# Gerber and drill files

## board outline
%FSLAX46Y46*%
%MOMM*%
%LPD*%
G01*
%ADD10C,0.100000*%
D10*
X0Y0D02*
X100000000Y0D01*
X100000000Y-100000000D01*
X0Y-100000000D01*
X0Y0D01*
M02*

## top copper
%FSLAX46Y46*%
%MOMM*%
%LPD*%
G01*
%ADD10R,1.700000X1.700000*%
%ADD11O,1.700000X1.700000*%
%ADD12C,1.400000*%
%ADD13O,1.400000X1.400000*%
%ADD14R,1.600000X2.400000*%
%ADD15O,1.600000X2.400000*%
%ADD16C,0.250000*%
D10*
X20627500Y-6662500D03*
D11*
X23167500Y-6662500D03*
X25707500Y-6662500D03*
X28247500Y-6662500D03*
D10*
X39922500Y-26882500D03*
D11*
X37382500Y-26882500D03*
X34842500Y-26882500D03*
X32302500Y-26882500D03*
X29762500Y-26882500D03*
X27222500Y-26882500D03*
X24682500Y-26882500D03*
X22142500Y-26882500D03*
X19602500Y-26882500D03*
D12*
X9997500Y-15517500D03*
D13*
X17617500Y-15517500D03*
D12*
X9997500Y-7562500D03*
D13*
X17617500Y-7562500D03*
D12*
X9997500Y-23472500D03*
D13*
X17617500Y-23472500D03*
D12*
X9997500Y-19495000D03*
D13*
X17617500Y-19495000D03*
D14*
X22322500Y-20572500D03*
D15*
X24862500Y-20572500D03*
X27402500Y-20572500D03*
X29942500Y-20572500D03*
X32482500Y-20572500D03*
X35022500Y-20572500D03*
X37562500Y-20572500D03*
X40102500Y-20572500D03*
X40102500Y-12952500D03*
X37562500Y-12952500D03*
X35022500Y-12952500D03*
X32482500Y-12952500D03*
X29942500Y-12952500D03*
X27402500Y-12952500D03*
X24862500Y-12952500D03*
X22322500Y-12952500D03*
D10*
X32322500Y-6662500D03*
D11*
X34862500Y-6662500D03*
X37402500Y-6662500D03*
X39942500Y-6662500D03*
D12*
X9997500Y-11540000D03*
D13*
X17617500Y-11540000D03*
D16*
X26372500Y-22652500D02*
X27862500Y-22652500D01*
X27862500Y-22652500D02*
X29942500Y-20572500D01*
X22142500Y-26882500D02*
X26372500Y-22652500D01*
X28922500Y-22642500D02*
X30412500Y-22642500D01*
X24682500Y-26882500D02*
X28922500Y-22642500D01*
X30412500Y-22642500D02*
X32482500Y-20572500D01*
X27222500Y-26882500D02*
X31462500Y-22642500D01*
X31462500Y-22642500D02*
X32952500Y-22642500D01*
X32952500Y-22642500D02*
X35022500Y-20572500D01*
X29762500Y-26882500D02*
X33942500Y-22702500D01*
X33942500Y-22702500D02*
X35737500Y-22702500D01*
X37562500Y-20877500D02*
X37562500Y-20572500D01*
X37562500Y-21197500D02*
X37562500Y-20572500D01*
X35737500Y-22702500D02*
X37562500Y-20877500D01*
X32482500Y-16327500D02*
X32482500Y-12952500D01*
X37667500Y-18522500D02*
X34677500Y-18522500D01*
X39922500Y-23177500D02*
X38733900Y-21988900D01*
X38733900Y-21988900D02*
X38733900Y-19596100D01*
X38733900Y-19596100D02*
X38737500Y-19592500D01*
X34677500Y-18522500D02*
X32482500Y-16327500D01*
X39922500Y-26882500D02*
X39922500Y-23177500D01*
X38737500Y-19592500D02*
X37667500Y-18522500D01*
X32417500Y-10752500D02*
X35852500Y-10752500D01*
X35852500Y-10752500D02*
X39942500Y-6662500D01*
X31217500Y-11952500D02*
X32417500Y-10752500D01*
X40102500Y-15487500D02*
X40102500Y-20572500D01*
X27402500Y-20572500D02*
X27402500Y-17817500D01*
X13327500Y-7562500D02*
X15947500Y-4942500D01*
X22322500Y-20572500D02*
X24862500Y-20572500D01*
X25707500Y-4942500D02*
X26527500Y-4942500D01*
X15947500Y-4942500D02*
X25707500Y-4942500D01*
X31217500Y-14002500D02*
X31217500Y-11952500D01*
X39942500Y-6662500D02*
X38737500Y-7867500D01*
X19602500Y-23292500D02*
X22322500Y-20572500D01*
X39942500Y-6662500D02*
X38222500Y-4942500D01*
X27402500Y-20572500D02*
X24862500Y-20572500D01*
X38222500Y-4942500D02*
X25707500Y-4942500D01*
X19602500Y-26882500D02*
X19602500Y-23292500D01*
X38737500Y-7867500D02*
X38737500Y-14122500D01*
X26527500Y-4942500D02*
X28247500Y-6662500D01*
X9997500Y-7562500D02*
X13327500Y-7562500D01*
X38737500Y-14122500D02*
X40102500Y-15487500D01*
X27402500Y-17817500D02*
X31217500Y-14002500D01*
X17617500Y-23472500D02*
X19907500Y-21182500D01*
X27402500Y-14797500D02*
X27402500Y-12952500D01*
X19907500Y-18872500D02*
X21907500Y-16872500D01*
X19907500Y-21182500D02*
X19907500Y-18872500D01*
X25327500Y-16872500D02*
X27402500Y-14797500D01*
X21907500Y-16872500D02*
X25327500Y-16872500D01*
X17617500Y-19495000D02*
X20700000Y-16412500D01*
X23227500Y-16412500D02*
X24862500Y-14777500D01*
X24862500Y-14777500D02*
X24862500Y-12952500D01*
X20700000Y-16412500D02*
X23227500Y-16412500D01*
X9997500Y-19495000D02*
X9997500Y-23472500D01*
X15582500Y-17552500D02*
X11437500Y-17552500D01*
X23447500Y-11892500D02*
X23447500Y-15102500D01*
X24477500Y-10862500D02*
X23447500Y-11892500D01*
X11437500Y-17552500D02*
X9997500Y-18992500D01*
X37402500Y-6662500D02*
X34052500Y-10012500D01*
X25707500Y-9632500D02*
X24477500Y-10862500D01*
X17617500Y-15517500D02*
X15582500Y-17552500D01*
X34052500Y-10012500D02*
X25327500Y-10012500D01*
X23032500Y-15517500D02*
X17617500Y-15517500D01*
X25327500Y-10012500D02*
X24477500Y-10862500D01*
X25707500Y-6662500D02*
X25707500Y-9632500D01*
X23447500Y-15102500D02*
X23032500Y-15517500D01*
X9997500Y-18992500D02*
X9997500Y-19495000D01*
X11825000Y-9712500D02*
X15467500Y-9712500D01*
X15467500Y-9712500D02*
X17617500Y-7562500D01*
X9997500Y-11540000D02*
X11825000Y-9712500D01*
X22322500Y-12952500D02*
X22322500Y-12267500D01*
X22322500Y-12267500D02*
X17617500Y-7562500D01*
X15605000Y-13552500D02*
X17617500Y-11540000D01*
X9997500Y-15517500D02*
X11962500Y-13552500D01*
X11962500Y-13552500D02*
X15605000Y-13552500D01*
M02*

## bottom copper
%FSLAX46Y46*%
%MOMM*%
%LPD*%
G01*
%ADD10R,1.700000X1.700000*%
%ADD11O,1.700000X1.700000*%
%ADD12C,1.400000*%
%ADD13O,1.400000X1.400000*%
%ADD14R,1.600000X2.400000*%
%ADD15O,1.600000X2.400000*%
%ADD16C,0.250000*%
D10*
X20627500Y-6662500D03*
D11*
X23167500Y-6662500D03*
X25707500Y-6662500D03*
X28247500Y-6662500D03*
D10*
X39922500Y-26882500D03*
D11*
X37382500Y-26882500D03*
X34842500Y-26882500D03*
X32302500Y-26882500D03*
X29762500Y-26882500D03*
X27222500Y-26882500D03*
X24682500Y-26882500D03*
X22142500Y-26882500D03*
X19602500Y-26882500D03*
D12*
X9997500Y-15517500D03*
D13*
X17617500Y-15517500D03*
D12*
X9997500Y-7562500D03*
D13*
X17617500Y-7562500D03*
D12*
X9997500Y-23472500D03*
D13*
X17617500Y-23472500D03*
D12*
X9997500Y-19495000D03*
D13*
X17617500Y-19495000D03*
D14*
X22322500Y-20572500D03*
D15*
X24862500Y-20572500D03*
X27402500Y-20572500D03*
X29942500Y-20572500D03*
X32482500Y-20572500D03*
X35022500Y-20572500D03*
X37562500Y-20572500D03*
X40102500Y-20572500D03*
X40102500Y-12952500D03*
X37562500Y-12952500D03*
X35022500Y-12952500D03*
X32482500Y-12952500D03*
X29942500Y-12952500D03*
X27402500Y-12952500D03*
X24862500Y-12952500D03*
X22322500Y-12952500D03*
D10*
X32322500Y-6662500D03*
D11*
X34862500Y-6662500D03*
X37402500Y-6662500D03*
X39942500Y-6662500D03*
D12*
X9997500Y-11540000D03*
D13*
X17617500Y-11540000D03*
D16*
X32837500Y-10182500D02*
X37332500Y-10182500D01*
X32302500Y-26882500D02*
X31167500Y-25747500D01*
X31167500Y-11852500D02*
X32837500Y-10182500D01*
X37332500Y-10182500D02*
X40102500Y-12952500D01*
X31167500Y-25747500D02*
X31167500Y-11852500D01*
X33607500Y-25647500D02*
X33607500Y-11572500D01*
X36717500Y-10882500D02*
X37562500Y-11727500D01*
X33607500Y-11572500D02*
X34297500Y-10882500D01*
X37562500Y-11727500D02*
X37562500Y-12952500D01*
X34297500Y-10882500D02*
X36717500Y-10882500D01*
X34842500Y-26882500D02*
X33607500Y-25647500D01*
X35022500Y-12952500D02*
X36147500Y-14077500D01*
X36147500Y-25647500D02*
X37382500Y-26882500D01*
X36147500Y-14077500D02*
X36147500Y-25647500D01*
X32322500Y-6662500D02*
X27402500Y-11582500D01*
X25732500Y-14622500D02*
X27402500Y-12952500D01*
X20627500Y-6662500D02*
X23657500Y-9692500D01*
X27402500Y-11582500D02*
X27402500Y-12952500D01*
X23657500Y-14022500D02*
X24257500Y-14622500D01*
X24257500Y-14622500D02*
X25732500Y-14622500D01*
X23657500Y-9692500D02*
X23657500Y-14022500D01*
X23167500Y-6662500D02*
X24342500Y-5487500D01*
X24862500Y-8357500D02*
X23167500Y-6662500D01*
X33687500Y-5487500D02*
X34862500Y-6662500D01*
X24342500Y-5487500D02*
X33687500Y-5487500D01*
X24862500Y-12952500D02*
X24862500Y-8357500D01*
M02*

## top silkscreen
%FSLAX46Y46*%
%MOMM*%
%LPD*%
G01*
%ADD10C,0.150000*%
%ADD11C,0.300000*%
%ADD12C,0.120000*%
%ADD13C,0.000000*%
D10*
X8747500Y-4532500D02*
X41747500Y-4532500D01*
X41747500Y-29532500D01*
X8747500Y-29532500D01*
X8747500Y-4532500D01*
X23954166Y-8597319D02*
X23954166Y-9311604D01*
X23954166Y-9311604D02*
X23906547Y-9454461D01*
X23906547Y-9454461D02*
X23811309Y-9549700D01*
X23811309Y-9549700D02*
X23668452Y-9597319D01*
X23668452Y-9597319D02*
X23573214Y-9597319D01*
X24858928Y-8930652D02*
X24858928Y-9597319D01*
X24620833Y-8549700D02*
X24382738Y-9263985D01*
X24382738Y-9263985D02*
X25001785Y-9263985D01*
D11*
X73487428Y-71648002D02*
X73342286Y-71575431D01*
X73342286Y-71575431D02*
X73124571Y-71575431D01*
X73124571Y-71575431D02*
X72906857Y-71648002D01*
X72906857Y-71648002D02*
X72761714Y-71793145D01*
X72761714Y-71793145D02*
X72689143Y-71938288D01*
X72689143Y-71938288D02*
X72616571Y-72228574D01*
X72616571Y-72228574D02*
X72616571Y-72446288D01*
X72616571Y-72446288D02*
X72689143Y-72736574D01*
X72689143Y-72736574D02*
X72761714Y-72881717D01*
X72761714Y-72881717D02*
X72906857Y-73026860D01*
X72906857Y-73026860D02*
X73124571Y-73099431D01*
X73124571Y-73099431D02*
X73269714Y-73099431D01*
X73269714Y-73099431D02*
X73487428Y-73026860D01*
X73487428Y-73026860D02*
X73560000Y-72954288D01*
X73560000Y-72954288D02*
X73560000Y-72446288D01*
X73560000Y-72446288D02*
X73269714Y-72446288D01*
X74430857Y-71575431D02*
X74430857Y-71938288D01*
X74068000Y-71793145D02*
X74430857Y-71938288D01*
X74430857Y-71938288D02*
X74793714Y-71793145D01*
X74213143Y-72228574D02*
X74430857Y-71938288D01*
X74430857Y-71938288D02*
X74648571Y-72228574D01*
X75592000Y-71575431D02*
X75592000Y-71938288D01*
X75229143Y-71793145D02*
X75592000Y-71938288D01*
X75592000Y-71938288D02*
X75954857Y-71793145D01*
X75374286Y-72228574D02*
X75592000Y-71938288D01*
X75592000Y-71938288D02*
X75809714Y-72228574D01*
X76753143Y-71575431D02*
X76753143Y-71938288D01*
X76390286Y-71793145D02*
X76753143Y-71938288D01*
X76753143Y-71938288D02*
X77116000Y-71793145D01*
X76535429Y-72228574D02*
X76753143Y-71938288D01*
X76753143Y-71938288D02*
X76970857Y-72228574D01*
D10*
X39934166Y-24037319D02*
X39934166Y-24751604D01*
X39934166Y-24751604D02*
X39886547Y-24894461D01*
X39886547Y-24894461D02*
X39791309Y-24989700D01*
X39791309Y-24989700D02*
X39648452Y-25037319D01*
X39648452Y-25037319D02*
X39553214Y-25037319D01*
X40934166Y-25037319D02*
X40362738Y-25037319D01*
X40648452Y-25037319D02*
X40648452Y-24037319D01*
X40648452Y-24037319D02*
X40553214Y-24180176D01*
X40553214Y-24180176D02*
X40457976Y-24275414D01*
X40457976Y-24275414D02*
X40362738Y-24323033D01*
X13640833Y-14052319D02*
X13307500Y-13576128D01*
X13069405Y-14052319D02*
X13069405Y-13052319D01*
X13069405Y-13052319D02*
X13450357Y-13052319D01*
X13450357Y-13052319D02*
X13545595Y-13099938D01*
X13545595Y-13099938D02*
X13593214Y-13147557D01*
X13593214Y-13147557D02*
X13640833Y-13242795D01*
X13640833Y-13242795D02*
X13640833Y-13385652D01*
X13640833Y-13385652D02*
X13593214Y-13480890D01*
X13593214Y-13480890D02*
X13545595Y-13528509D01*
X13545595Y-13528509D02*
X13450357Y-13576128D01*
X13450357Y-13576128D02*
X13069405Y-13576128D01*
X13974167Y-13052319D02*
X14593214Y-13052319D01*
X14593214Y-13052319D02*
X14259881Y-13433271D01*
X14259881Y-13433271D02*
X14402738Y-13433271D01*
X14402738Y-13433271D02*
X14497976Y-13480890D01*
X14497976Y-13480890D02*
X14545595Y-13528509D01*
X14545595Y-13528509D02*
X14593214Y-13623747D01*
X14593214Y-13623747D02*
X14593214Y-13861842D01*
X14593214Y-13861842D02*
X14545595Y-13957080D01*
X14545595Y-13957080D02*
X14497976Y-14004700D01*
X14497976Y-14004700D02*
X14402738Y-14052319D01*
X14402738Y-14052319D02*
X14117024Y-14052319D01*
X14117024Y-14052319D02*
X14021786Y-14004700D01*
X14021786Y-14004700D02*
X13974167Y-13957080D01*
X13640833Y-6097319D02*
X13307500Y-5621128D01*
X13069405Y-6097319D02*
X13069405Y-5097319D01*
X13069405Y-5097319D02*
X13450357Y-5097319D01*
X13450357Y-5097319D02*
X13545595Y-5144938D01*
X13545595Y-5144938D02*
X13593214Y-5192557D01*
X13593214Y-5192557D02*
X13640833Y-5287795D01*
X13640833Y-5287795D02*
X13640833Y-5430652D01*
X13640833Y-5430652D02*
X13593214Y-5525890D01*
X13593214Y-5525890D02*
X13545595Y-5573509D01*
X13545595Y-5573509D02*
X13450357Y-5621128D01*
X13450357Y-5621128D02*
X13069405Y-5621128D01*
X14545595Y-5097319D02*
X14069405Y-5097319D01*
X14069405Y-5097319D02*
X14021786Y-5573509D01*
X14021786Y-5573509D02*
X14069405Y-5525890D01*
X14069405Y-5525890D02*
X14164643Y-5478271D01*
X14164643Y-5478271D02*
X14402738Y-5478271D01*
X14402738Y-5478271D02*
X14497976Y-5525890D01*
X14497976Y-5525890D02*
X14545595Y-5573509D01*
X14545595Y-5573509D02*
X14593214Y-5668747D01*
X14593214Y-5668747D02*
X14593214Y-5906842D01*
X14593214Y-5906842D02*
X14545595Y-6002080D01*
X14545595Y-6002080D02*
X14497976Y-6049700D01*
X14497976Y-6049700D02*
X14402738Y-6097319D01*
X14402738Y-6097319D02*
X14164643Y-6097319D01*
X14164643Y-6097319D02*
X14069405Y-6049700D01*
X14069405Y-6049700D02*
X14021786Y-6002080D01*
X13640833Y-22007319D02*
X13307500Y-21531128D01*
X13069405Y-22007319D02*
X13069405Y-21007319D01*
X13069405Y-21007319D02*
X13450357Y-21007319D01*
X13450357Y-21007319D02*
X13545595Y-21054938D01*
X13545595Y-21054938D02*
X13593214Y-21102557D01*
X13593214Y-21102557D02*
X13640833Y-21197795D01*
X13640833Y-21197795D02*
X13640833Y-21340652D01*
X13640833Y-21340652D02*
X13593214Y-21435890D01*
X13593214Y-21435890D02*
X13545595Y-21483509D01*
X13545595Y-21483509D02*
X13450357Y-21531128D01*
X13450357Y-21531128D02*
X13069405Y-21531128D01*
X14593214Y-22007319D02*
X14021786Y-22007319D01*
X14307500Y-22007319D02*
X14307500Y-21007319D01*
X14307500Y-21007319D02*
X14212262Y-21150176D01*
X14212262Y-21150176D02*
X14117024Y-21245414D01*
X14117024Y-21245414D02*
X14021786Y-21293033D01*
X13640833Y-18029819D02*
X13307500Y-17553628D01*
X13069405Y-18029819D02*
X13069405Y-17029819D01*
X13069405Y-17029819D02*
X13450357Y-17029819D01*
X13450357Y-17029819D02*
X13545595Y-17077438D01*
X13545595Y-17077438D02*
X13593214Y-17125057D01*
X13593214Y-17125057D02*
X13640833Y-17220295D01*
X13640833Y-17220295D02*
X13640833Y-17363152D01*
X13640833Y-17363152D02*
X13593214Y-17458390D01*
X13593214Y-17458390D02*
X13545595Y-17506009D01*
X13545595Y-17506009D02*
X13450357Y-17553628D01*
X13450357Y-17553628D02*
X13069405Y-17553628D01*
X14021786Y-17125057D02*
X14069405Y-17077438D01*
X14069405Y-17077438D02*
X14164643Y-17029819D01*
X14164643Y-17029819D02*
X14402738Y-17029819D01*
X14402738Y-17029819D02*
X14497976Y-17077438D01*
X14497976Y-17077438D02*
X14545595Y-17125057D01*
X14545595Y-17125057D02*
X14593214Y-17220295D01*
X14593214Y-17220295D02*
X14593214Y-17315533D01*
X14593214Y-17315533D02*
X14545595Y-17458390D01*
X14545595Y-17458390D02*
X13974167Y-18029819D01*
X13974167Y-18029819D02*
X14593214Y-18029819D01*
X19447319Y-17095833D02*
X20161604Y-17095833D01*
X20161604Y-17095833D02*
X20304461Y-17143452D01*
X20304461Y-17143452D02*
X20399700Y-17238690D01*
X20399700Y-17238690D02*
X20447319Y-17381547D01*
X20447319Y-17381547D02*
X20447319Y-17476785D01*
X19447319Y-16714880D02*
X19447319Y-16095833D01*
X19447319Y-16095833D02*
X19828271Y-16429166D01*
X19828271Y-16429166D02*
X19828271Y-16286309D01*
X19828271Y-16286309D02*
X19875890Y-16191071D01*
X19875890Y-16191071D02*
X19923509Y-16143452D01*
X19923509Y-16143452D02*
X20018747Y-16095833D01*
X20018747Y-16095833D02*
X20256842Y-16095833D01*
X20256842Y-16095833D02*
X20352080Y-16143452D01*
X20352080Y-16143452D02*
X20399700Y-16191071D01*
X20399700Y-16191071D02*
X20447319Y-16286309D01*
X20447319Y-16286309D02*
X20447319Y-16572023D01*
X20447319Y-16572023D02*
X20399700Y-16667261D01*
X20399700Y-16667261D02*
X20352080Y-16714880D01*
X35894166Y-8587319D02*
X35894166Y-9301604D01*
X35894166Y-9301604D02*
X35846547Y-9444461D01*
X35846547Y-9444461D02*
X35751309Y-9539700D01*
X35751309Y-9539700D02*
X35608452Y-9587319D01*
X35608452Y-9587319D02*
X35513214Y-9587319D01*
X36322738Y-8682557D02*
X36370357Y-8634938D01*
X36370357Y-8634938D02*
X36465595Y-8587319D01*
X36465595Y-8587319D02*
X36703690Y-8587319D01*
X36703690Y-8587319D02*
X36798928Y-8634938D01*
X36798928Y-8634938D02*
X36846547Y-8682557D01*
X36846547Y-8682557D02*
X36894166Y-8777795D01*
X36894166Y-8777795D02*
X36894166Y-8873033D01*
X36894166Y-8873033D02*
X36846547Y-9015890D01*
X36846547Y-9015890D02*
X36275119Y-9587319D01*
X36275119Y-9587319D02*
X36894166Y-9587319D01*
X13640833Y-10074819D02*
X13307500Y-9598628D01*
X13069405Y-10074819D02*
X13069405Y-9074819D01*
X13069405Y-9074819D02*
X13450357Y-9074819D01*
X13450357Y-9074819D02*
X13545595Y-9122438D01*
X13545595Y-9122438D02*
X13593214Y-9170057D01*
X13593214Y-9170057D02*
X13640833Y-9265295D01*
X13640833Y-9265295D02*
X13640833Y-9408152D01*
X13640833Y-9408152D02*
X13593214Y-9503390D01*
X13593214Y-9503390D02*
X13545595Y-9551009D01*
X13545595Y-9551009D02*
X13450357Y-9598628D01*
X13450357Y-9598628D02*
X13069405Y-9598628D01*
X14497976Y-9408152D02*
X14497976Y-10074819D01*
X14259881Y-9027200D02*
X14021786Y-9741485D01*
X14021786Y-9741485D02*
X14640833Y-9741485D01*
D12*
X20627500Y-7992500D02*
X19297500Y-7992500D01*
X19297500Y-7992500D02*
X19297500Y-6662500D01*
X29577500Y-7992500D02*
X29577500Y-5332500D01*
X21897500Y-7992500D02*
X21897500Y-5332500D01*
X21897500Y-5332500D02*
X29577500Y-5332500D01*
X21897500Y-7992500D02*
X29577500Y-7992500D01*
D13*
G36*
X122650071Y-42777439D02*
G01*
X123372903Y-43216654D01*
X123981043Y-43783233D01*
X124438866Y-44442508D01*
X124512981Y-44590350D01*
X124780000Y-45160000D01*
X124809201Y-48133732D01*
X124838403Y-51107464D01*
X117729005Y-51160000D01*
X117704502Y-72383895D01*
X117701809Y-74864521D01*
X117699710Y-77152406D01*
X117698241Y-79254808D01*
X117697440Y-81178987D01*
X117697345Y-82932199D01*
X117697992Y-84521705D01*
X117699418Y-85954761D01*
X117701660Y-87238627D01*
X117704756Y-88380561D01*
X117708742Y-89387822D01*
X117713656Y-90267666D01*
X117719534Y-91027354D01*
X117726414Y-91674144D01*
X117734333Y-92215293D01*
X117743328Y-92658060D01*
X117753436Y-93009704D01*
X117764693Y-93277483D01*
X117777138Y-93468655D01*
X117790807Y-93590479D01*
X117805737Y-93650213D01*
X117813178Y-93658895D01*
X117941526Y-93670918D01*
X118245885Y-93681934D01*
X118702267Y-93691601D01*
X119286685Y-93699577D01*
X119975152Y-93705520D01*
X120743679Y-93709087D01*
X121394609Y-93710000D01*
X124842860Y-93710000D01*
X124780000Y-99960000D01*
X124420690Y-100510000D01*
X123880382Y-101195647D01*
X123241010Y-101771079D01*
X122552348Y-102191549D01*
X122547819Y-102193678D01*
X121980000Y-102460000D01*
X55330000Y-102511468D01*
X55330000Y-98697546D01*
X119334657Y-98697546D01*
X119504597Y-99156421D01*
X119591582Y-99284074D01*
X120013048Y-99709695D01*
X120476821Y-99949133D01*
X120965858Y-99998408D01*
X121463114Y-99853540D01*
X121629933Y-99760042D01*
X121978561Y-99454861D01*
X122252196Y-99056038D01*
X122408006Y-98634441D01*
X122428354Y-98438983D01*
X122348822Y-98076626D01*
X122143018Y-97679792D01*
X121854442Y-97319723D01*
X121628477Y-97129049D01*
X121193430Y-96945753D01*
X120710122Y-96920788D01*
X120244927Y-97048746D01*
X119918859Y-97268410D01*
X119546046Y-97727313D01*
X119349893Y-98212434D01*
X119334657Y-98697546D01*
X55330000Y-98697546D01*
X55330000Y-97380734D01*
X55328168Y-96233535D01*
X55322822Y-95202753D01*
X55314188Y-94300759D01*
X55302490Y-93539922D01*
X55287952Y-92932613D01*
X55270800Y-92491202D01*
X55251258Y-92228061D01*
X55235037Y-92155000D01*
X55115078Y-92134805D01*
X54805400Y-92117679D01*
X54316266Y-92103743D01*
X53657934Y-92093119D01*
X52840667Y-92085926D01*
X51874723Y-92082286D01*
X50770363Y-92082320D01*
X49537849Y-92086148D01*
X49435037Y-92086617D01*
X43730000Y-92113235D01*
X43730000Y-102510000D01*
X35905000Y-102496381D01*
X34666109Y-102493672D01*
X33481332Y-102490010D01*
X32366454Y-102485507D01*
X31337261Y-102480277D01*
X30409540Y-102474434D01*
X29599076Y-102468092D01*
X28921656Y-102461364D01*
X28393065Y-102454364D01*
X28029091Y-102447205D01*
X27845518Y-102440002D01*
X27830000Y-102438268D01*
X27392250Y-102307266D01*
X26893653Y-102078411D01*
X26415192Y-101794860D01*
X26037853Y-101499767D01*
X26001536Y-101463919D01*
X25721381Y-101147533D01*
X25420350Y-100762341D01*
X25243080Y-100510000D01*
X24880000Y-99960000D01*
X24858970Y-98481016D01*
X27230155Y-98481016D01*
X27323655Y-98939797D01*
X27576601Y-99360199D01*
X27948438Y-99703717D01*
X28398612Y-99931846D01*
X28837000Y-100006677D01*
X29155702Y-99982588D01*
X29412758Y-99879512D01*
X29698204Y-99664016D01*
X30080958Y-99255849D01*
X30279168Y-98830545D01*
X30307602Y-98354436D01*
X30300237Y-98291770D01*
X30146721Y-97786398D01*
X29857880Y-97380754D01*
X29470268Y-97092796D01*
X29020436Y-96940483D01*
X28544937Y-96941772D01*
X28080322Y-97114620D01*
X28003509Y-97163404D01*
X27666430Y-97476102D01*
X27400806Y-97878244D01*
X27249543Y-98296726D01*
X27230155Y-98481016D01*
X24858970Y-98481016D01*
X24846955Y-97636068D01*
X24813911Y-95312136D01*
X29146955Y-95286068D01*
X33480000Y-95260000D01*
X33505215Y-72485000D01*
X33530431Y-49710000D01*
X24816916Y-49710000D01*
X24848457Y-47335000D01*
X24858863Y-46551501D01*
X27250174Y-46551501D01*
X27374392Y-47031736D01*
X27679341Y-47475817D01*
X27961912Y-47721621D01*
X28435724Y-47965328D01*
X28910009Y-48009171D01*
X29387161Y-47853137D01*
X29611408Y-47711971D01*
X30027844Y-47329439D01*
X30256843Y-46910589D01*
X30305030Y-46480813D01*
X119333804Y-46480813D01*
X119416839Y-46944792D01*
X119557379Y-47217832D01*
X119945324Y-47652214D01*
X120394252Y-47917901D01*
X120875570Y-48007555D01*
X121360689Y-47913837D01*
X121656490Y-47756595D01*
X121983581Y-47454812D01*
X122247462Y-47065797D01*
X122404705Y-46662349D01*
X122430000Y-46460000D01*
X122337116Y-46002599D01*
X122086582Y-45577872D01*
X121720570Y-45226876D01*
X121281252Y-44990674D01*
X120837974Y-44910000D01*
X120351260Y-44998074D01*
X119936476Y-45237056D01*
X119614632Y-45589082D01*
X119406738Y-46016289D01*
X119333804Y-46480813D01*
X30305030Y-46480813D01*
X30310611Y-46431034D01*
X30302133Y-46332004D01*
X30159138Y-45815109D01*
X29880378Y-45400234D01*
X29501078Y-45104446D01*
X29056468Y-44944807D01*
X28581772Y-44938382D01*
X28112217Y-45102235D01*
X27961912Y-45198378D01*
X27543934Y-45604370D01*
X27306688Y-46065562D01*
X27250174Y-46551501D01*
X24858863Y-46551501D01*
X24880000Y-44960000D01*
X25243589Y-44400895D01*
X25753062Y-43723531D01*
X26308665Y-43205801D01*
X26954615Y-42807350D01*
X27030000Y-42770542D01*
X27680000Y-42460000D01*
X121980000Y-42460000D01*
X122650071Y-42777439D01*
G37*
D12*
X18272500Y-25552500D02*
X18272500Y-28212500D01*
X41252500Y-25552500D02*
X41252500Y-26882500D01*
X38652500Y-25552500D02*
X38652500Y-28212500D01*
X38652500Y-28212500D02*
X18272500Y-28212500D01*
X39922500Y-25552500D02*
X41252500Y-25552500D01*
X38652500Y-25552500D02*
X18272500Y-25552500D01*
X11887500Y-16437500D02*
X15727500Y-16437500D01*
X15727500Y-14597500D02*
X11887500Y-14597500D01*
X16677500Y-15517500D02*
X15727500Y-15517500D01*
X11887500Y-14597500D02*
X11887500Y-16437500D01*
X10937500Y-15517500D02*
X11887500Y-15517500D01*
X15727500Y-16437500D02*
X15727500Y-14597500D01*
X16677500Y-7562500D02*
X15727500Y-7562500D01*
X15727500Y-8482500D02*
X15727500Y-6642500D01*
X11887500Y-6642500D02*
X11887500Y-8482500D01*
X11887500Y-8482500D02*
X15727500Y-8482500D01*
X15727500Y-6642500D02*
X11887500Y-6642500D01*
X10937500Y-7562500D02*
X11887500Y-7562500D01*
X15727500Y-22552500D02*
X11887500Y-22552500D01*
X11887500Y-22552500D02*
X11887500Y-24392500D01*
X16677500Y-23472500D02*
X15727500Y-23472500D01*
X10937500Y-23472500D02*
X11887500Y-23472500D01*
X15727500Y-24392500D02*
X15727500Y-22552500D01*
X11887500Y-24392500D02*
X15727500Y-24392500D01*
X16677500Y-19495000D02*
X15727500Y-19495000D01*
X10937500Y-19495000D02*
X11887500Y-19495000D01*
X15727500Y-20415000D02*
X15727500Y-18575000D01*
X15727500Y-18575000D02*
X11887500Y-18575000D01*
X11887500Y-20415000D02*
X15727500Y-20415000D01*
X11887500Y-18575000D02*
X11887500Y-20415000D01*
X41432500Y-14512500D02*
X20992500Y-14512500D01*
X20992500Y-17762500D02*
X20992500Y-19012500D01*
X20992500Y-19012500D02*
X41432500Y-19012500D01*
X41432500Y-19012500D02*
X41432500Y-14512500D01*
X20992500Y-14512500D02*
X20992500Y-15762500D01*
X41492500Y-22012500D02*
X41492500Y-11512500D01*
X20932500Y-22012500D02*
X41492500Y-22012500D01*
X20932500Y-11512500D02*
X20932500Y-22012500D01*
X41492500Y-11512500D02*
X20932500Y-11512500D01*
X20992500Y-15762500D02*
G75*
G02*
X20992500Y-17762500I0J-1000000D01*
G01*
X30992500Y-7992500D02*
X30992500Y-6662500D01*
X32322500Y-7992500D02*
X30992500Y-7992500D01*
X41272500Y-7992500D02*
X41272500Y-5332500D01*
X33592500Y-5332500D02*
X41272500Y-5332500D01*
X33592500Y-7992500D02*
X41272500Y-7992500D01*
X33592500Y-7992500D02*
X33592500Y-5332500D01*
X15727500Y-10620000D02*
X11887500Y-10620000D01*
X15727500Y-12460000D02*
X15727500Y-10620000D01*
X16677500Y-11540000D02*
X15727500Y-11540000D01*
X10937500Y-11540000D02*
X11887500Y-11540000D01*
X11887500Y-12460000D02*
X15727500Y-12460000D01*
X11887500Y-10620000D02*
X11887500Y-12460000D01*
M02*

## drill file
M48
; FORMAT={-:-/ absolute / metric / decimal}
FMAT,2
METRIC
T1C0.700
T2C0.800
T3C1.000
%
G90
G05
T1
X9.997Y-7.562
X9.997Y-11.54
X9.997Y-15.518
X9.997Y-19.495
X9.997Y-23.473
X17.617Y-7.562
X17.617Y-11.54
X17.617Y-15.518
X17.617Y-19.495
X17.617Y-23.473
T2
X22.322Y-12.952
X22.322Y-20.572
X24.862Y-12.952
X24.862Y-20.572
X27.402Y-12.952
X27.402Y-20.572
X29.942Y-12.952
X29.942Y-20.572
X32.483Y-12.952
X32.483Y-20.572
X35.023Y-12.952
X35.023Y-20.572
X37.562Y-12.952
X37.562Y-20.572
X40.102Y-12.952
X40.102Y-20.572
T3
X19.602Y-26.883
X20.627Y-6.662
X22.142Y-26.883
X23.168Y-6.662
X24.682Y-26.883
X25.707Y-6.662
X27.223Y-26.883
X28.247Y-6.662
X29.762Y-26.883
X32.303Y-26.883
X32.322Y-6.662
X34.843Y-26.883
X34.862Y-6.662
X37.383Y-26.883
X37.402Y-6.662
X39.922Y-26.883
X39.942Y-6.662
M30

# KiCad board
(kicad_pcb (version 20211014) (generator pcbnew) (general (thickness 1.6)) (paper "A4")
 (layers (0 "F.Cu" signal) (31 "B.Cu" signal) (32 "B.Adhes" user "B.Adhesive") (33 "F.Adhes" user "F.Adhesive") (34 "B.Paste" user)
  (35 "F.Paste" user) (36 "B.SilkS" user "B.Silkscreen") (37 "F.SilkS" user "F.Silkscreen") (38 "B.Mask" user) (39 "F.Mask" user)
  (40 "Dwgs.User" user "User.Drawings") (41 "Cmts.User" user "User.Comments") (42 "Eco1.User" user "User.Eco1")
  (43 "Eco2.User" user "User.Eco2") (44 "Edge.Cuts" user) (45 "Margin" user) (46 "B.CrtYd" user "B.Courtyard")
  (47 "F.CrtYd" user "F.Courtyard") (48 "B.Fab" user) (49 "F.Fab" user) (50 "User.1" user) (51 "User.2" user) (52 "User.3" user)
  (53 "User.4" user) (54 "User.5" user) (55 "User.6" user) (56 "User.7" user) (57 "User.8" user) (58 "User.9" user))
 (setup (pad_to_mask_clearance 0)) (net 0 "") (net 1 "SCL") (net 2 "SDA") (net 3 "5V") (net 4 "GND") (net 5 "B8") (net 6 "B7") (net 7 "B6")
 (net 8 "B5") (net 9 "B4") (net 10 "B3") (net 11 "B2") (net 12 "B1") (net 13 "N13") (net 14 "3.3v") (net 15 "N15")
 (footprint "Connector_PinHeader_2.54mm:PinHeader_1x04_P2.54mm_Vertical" (layer "F.Cu") (at 20.6275 6.6625 90)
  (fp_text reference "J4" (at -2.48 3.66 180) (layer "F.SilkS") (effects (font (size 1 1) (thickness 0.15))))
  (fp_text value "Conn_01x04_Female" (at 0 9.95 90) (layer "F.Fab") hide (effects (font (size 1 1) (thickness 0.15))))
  (fp_line (start -1.33 0) (end -1.33 -1.33) (layer "F.SilkS") (width 0.12))
  (fp_line (start -1.33 -1.33) (end 0 -1.33) (layer "F.SilkS") (width 0.12))
  (fp_line (start -1.33 8.95) (end 1.33 8.95) (layer "F.SilkS") (width 0.12))
  (fp_line (start -1.33 1.27) (end 1.33 1.27) (layer "F.SilkS") (width 0.12))
  (fp_line (start 1.33 1.27) (end 1.33 8.95) (layer "F.SilkS") (width 0.12))
  (fp_line (start -1.33 1.27) (end -1.33 8.95) (layer "F.SilkS") (width 0.12))
  (pad "1" thru_hole rect (at 0 0 90) (size 1.7 1.7) (drill 1) (layers *.Cu *.Mask) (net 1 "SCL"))
  (pad "2" thru_hole oval (at 0 2.54 90) (size 1.7 1.7) (drill 1) (layers *.Cu *.Mask) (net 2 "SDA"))
  (pad "3" thru_hole oval (at 0 5.08 90) (size 1.7 1.7) (drill 1) (layers *.Cu *.Mask) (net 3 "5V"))
  (pad "4" thru_hole oval (at 0 7.62 90) (size 1.7 1.7) (drill 1) (layers *.Cu *.Mask) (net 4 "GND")))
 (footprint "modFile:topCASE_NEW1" (layer "F.Cu") (at 74.83 72.41)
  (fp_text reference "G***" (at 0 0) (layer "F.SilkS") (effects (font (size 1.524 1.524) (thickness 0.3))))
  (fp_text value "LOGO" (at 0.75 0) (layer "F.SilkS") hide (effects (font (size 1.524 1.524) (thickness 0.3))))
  (fp_poly
   (pts (xy 47.820071 -29.632561) (xy 48.542903 -29.193346) (xy 49.151043 -28.626767) (xy 49.608866 -27.967492) (xy 49.682981 -27.81965)
    (xy 49.95 -27.25) (xy 49.979201 -24.276268) (xy 50.008403 -21.302536) (xy 42.899005 -21.25) (xy 42.874502 -0.026105)
    (xy 42.871809 2.454521) (xy 42.86971 4.742406) (xy 42.868241 6.844808) (xy 42.86744 8.768987) (xy 42.867345 10.522199)
    (xy 42.867992 12.111705) (xy 42.869418 13.544761) (xy 42.87166 14.828627) (xy 42.874756 15.970561) (xy 42.878742 16.977822)
    (xy 42.883656 17.857666) (xy 42.889534 18.617354) (xy 42.896414 19.264144) (xy 42.904333 19.805293) (xy 42.913328 20.24806)
    (xy 42.923436 20.599704) (xy 42.934693 20.867483) (xy 42.947138 21.058655) (xy 42.960807 21.180479) (xy 42.975737 21.240213)
    (xy 42.983178 21.248895) (xy 43.111526 21.260918) (xy 43.415885 21.271934) (xy 43.872267 21.281601) (xy 44.456685 21.289577)
    (xy 45.145152 21.29552) (xy 45.913679 21.299087) (xy 46.564609 21.3) (xy 50.01286 21.3) (xy 49.95 27.55) (xy 49.59069 28.1)
    (xy 49.050382 28.785647) (xy 48.41101 29.361079) (xy 47.722348 29.781549) (xy 47.717819 29.783678) (xy 47.15 30.05) (xy -19.5 30.101468)
    (xy -19.5 26.287546) (xy 44.504657 26.287546) (xy 44.674597 26.746421) (xy 44.761582 26.874074) (xy 45.183048 27.299695)
    (xy 45.646821 27.539133) (xy 46.135858 27.588408) (xy 46.633114 27.44354) (xy 46.799933 27.350042) (xy 47.148561 27.044861)
    (xy 47.422196 26.646038) (xy 47.578006 26.224441) (xy 47.598354 26.028983) (xy 47.518822 25.666626) (xy 47.313018 25.269792)
    (xy 47.024442 24.909723) (xy 46.798477 24.719049) (xy 46.36343 24.535753) (xy 45.880122 24.510788) (xy 45.414927 24.638746)
    (xy 45.088859 24.85841) (xy 44.716046 25.317313) (xy 44.519893 25.802434) (xy 44.504657 26.287546) (xy -19.5 26.287546)
    (xy -19.5 24.970734) (xy -19.501832 23.823535) (xy -19.507178 22.792753) (xy -19.515812 21.890759) (xy -19.52751 21.129922)
    (xy -19.542048 20.522613) (xy -19.5592 20.081202) (xy -19.578742 19.818061) (xy -19.594963 19.745) (xy -19.714922 19.724805)
    (xy -20.0246 19.707679) (xy -20.513734 19.693743) (xy -21.172066 19.683119) (xy -21.989333 19.675926) (xy -22.955277 19.672286)
    (xy -24.059637 19.67232) (xy -25.292151 19.676148) (xy -25.394963 19.676617) (xy -31.1 19.703235) (xy -31.1 30.1) (xy -38.925 30.086381)
    (xy -40.163891 30.083672) (xy -41.348668 30.08001) (xy -42.463546 30.075507) (xy -43.492739 30.070277) (xy -44.42046 30.064434)
    (xy -45.230924 30.058092) (xy -45.908344 30.051364) (xy -46.436935 30.044364) (xy -46.800909 30.037205) (xy -46.984482 30.030002)
    (xy -47 30.028268) (xy -47.43775 29.897266) (xy -47.936347 29.668411) (xy -48.414808 29.38486) (xy -48.792147 29.089767)
    (xy -48.828464 29.053919) (xy -49.108619 28.737533) (xy -49.40965 28.352341) (xy -49.58692 28.1) (xy -49.95 27.55)
    (xy -49.97103 26.071016) (xy -47.599845 26.071016) (xy -47.506345 26.529797) (xy -47.253399 26.950199) (xy -46.881562 27.293717)
    (xy -46.431388 27.521846) (xy -45.993 27.596677) (xy -45.674298 27.572588) (xy -45.417242 27.469512) (xy -45.131796 27.254016)
    (xy -44.749042 26.845849) (xy -44.550832 26.420545) (xy -44.522398 25.944436) (xy -44.529763 25.88177) (xy -44.683279 25.376398)
    (xy -44.97212 24.970754) (xy -45.359732 24.682796) (xy -45.809564 24.530483) (xy -46.285063 24.531772) (xy -46.749678 24.70462)
    (xy -46.826491 24.753404) (xy -47.16357 25.066102) (xy -47.429194 25.468244) (xy -47.580457 25.886726) (xy -47.599845 26.071016)
    (xy -49.97103 26.071016) (xy -49.983045 25.226068) (xy -50.016089 22.902136) (xy -45.683045 22.876068) (xy -41.35 22.85)
    (xy -41.324785 0.075) (xy -41.299569 -22.7) (xy -50.013084 -22.7) (xy -49.981543 -25.075) (xy -49.971137 -25.858499)
    (xy -47.579826 -25.858499) (xy -47.455608 -25.378264) (xy -47.150659 -24.934183) (xy -46.868088 -24.688379) (xy -46.394276 -24.444672)
    (xy -45.919991 -24.400829) (xy -45.442839 -24.556863) (xy -45.218592 -24.698029) (xy -44.802156 -25.080561) (xy -44.573157 -25.499411)
    (xy -44.52497 -25.929187) (xy 44.503804 -25.929187) (xy 44.586839 -25.465208) (xy 44.727379 -25.192168) (xy 45.115324 -24.757786)
    (xy 45.564252 -24.492099) (xy 46.04557 -24.402445) (xy 46.530689 -24.496163) (xy 46.82649 -24.653405) (xy 47.153581 -24.955188)
    (xy 47.417462 -25.344203) (xy 47.574705 -25.747651) (xy 47.6 -25.95) (xy 47.507116 -26.407401) (xy 47.256582 -26.832128)
    (xy 46.89057 -27.183124) (xy 46.451252 -27.419326) (xy 46.007974 -27.5) (xy 45.52126 -27.411926) (xy 45.106476 -27.172944)
    (xy 44.784632 -26.820918) (xy 44.576738 -26.393711) (xy 44.503804 -25.929187) (xy -44.52497 -25.929187) (xy -44.519389 -25.978966)
    (xy -44.527867 -26.077996) (xy -44.670862 -26.594891) (xy -44.949622 -27.009766) (xy -45.328922 -27.305554) (xy -45.773532 -27.465193)
    (xy -46.248228 -27.471618) (xy -46.717783 -27.307765) (xy -46.868088 -27.211622) (xy -47.286066 -26.80563) (xy -47.523312 -26.344438)
    (xy -47.579826 -25.858499) (xy -49.971137 -25.858499) (xy -49.95 -27.45) (xy -49.586411 -28.009105) (xy -49.076938 -28.686469)
    (xy -48.521335 -29.204199) (xy -47.875385 -29.60265) (xy -47.8 -29.639458) (xy -47.15 -29.95) (xy 47.15 -29.95))
   (layer "F.SilkS") (width 0) (fill solid)))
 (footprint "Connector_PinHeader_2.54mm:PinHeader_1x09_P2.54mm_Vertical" (layer "F.Cu") (at 39.9225 26.8825 -90)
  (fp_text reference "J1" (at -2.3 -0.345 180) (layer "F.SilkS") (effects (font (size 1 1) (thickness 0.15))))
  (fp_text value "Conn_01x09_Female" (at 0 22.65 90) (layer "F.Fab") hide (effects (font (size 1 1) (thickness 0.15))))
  (fp_line (start -1.33 21.65) (end 1.33 21.65) (layer "F.SilkS") (width 0.12))
  (fp_line (start -1.33 -1.33) (end 0 -1.33) (layer "F.SilkS") (width 0.12))
  (fp_line (start -1.33 1.27) (end 1.33 1.27) (layer "F.SilkS") (width 0.12))
  (fp_line (start 1.33 1.27) (end 1.33 21.65) (layer "F.SilkS") (width 0.12))
  (fp_line (start -1.33 0) (end -1.33 -1.33) (layer "F.SilkS") (width 0.12))
  (fp_line (start -1.33 1.27) (end -1.33 21.65) (layer "F.SilkS") (width 0.12))
  (pad "1" thru_hole rect (at 0 0 270) (size 1.7 1.7) (drill 1) (layers *.Cu *.Mask) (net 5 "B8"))
  (pad "2" thru_hole oval (at 0 2.54 270) (size 1.7 1.7) (drill 1) (layers *.Cu *.Mask) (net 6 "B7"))
  (pad "3" thru_hole oval (at 0 5.08 270) (size 1.7 1.7) (drill 1) (layers *.Cu *.Mask) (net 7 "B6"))
  (pad "4" thru_hole oval (at 0 7.62 270) (size 1.7 1.7) (drill 1) (layers *.Cu *.Mask) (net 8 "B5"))
  (pad "5" thru_hole oval (at 0 10.16 270) (size 1.7 1.7) (drill 1) (layers *.Cu *.Mask) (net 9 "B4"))
  (pad "6" thru_hole oval (at 0 12.7 270) (size 1.7 1.7) (drill 1) (layers *.Cu *.Mask) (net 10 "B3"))
  (pad "7" thru_hole oval (at 0 15.24 270) (size 1.7 1.7) (drill 1) (layers *.Cu *.Mask) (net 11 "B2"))
  (pad "8" thru_hole oval (at 0 17.78 270) (size 1.7 1.7) (drill 1) (layers *.Cu *.Mask) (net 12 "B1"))
  (pad "9" thru_hole oval (at 0 20.32 270) (size 1.7 1.7) (drill 1) (layers *.Cu *.Mask) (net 4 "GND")))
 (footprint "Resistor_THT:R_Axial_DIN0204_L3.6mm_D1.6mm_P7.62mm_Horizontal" (layer "F.Cu") (at 9.9975 15.5175)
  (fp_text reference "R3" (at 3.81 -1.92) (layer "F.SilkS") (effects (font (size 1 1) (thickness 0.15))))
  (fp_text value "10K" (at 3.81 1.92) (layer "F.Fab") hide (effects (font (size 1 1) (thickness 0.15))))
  (fp_line (start 1.89 0.92) (end 5.73 0.92) (layer "F.SilkS") (width 0.12))
  (fp_line (start 5.73 -0.92) (end 1.89 -0.92) (layer "F.SilkS") (width 0.12))
  (fp_line (start 6.68 0) (end 5.73 0) (layer "F.SilkS") (width 0.12))
  (fp_line (start 1.89 -0.92) (end 1.89 0.92) (layer "F.SilkS") (width 0.12))
  (fp_line (start 0.94 0) (end 1.89 0) (layer "F.SilkS") (width 0.12))
  (fp_line (start 5.73 0.92) (end 5.73 -0.92) (layer "F.SilkS") (width 0.12))
  (pad "1" thru_hole circle (at 0 0) (size 1.4 1.4) (drill 0.7) (layers *.Cu *.Mask) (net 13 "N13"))
  (pad "2" thru_hole oval (at 7.62 0) (size 1.4 1.4) (drill 0.7) (layers *.Cu *.Mask) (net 3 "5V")))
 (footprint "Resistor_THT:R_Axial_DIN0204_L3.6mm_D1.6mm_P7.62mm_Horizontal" (layer "F.Cu") (at 9.9975 7.5625)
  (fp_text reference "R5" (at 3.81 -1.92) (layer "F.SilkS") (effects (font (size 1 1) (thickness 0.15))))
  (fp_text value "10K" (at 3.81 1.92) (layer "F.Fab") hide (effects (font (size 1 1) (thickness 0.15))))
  (fp_line (start 6.68 0) (end 5.73 0) (layer "F.SilkS") (width 0.12))
  (fp_line (start 5.73 0.92) (end 5.73 -0.92) (layer "F.SilkS") (width 0.12))
  (fp_line (start 1.89 -0.92) (end 1.89 0.92) (layer "F.SilkS") (width 0.12))
  (fp_line (start 1.89 0.92) (end 5.73 0.92) (layer "F.SilkS") (width 0.12))
  (fp_line (start 5.73 -0.92) (end 1.89 -0.92) (layer "F.SilkS") (width 0.12))
  (fp_line (start 0.94 0) (end 1.89 0) (layer "F.SilkS") (width 0.12))
  (pad "1" thru_hole circle (at 0 0) (size 1.4 1.4) (drill 0.7) (layers *.Cu *.Mask) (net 4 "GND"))
  (pad "2" thru_hole oval (at 7.62 0) (size 1.4 1.4) (drill 0.7) (layers *.Cu *.Mask) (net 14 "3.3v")))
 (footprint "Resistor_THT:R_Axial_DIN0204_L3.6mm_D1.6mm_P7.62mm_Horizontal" (layer "F.Cu") (at 9.9975 23.4725)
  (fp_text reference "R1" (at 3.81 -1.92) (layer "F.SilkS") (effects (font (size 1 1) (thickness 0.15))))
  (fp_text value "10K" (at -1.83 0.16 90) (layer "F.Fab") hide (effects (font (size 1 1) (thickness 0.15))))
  (fp_line (start 5.73 -0.92) (end 1.89 -0.92) (layer "F.SilkS") (width 0.12))
  (fp_line (start 1.89 -0.92) (end 1.89 0.92) (layer "F.SilkS") (width 0.12))
  (fp_line (start 6.68 0) (end 5.73 0) (layer "F.SilkS") (width 0.12))
  (fp_line (start 0.94 0) (end 1.89 0) (layer "F.SilkS") (width 0.12))
  (fp_line (start 5.73 0.92) (end 5.73 -0.92) (layer "F.SilkS") (width 0.12))
  (fp_line (start 1.89 0.92) (end 5.73 0.92) (layer "F.SilkS") (width 0.12))
  (pad "1" thru_hole circle (at 0 0) (size 1.4 1.4) (drill 0.7) (layers *.Cu *.Mask) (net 3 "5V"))
  (pad "2" thru_hole oval (at 7.62 0) (size 1.4 1.4) (drill 0.7) (layers *.Cu *.Mask) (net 1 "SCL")))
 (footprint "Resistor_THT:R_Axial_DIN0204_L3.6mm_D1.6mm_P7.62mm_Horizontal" (layer "F.Cu") (at 9.9975 19.495)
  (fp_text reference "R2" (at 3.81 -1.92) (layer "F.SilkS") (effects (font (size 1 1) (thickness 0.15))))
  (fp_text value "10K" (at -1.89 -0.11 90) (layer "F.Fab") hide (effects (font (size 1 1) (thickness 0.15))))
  (fp_line (start 6.68 0) (end 5.73 0) (layer "F.SilkS") (width 0.12))
  (fp_line (start 0.94 0) (end 1.89 0) (layer "F.SilkS") (width 0.12))
  (fp_line (start 5.73 0.92) (end 5.73 -0.92) (layer "F.SilkS") (width 0.12))
  (fp_line (start 5.73 -0.92) (end 1.89 -0.92) (layer "F.SilkS") (width 0.12))
  (fp_line (start 1.89 0.92) (end 5.73 0.92) (layer "F.SilkS") (width 0.12))
  (fp_line (start 1.89 -0.92) (end 1.89 0.92) (layer "F.SilkS") (width 0.12))
  (pad "1" thru_hole circle (at 0 0) (size 1.4 1.4) (drill 0.7) (layers *.Cu *.Mask) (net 3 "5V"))
  (pad "2" thru_hole oval (at 7.62 0) (size 1.4 1.4) (drill 0.7) (layers *.Cu *.Mask) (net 2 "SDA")))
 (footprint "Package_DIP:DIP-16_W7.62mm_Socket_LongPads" (layer "F.Cu") (at 22.3225 20.5725 90)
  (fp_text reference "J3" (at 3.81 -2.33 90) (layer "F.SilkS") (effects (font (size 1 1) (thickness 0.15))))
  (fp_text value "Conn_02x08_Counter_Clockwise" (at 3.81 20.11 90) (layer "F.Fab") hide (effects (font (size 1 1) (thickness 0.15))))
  (fp_line (start 6.06 19.11) (end 6.06 -1.33) (layer "F.SilkS") (width 0.12))
  (fp_line (start 2.81 -1.33) (end 1.56 -1.33) (layer "F.SilkS") (width 0.12))
  (fp_line (start 1.56 -1.33) (end 1.56 19.11) (layer "F.SilkS") (width 0.12))
  (fp_line (start 1.56 19.11) (end 6.06 19.11) (layer "F.SilkS") (width 0.12))
  (fp_line (start 6.06 -1.33) (end 4.81 -1.33) (layer "F.SilkS") (width 0.12))
  (fp_line (start -1.44 19.17) (end 9.06 19.17) (layer "F.SilkS") (width 0.12))
  (fp_line (start -1.44 -1.39) (end -1.44 19.17) (layer "F.SilkS") (width 0.12))
  (fp_line (start 9.06 -1.39) (end -1.44 -1.39) (layer "F.SilkS") (width 0.12))
  (fp_line (start 9.06 19.17) (end 9.06 -1.39) (layer "F.SilkS") (width 0.12))
  (fp_arc (start 4.81 -1.33) (mid 3.81 -0.33) (end 2.81 -1.33) (layer "F.SilkS") (width 0.12))
  (pad "1" thru_hole rect (at 0 0 90) (size 2.4 1.6) (drill 0.8) (layers *.Cu *.Mask) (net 4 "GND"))
  (pad "2" thru_hole oval (at 0 2.54 90) (size 2.4 1.6) (drill 0.8) (layers *.Cu *.Mask) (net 4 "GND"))
  (pad "3" thru_hole oval (at 0 5.08 90) (size 2.4 1.6) (drill 0.8) (layers *.Cu *.Mask) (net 4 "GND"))
  (pad "4" thru_hole oval (at 0 7.62 90) (size 2.4 1.6) (drill 0.8) (layers *.Cu *.Mask) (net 12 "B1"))
  (pad "5" thru_hole oval (at 0 10.16 90) (size 2.4 1.6) (drill 0.8) (layers *.Cu *.Mask) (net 11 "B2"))
  (pad "6" thru_hole oval (at 0 12.7 90) (size 2.4 1.6) (drill 0.8) (layers *.Cu *.Mask) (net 10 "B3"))
  (pad "7" thru_hole oval (at 0 15.24 90) (size 2.4 1.6) (drill 0.8) (layers *.Cu *.Mask) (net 9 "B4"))
  (pad "8" thru_hole oval (at 0 17.78 90) (size 2.4 1.6) (drill 0.8) (layers *.Cu *.Mask) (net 4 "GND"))
  (pad "9" thru_hole oval (at 7.62 17.78 90) (size 2.4 1.6) (drill 0.8) (layers *.Cu *.Mask) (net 8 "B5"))
  (pad "10" thru_hole oval (at 7.62 15.24 90) (size 2.4 1.6) (drill 0.8) (layers *.Cu *.Mask) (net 7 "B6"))
  (pad "11" thru_hole oval (at 7.62 12.7 90) (size 2.4 1.6) (drill 0.8) (layers *.Cu *.Mask) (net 6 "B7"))
  (pad "12" thru_hole oval (at 7.62 10.16 90) (size 2.4 1.6) (drill 0.8) (layers *.Cu *.Mask) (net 5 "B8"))
  (pad "13" thru_hole oval (at 7.62 7.62 90) (size 2.4 1.6) (drill 0.8) (layers *.Cu *.Mask) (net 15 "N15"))
  (pad "14" thru_hole oval (at 7.62 5.08 90) (size 2.4 1.6) (drill 0.8) (layers *.Cu *.Mask) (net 1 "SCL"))
  (pad "15" thru_hole oval (at 7.62 2.54 90) (size 2.4 1.6) (drill 0.8) (layers *.Cu *.Mask) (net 2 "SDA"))
  (pad "16" thru_hole oval (at 7.62 0 90) (size 2.4 1.6) (drill 0.8) (layers *.Cu *.Mask) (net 14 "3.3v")))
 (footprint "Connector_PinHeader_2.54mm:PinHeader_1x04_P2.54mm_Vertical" (layer "F.Cu") (at 32.3225 6.6625 90)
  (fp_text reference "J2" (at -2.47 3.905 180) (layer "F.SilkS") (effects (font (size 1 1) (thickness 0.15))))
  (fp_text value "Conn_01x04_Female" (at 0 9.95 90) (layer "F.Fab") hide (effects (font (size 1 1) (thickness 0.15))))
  (fp_line (start -1.33 -1.33) (end 0 -1.33) (layer "F.SilkS") (width 0.12))
  (fp_line (start -1.33 0) (end -1.33 -1.33) (layer "F.SilkS") (width 0.12))
  (fp_line (start -1.33 8.95) (end 1.33 8.95) (layer "F.SilkS") (width 0.12))
  (fp_line (start 1.33 1.27) (end 1.33 8.95) (layer "F.SilkS") (width 0.12))
  (fp_line (start -1.33 1.27) (end -1.33 8.95) (layer "F.SilkS") (width 0.12))
  (fp_line (start -1.33 1.27) (end 1.33 1.27) (layer "F.SilkS") (width 0.12))
  (pad "1" thru_hole rect (at 0 0 90) (size 1.7 1.7) (drill 1) (layers *.Cu *.Mask) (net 1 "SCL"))
  (pad "2" thru_hole oval (at 0 2.54 90) (size 1.7 1.7) (drill 1) (layers *.Cu *.Mask) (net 2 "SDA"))
  (pad "3" thru_hole oval (at 0 5.08 90) (size 1.7 1.7) (drill 1) (layers *.Cu *.Mask) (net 3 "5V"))
  (pad "4" thru_hole oval (at 0 7.62 90) (size 1.7 1.7) (drill 1) (layers *.Cu *.Mask) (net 4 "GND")))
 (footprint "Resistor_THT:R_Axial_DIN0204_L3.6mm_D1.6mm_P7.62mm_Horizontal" (layer "F.Cu") (at 9.9975 11.54)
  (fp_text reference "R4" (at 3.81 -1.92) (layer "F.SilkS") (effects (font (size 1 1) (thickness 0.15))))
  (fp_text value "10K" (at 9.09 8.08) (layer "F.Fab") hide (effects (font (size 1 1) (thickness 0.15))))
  (fp_line (start 5.73 -0.92) (end 1.89 -0.92) (layer "F.SilkS") (width 0.12))
  (fp_line (start 5.73 0.92) (end 5.73 -0.92) (layer "F.SilkS") (width 0.12))
  (fp_line (start 6.68 0) (end 5.73 0) (layer "F.SilkS") (width 0.12))
  (fp_line (start 0.94 0) (end 1.89 0) (layer "F.SilkS") (width 0.12))
  (fp_line (start 1.89 0.92) (end 5.73 0.92) (layer "F.SilkS") (width 0.12))
  (fp_line (start 1.89 -0.92) (end 1.89 0.92) (layer "F.SilkS") (width 0.12))
  (pad "1" thru_hole circle (at 0 0) (size 1.4 1.4) (drill 0.7) (layers *.Cu *.Mask) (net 14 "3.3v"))
  (pad "2" thru_hole oval (at 7.62 0) (size 1.4 1.4) (drill 0.7) (layers *.Cu *.Mask) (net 13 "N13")))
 (gr_rect (start 41.7475 29.5325) (end 8.7475 4.5325) (layer "F.SilkS") (width 0.15) (fill none))
 (gr_rect (start 0 0) (end 100 100) (layer "Edge.Cuts") (width 0.1) (fill none))
 (segment (start 26.3725 22.6525) (end 27.8625 22.6525) (width 0.25) (layer "F.Cu") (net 12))
 (segment (start 27.8625 22.6525) (end 29.9425 20.5725) (width 0.25) (layer "F.Cu") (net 12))
 (segment (start 22.1425 26.8825) (end 26.3725 22.6525) (width 0.25) (layer "F.Cu") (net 12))
 (segment (start 28.9225 22.6425) (end 30.4125 22.6425) (width 0.25) (layer "F.Cu") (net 11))
 (segment (start 24.6825 26.8825) (end 28.9225 22.6425) (width 0.25) (layer "F.Cu") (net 11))
 (segment (start 30.4125 22.6425) (end 32.4825 20.5725) (width 0.25) (layer "F.Cu") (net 11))
 (segment (start 27.2225 26.8825) (end 31.4625 22.6425) (width 0.25) (layer "F.Cu") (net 10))
 (segment (start 31.4625 22.6425) (end 32.9525 22.6425) (width 0.25) (layer "F.Cu") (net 10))
 (segment (start 32.9525 22.6425) (end 35.0225 20.5725) (width 0.25) (layer "F.Cu") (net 10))
 (segment (start 29.7625 26.8825) (end 33.9425 22.7025) (width 0.25) (layer "F.Cu") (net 9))
 (segment (start 33.9425 22.7025) (end 35.7375 22.7025) (width 0.25) (layer "F.Cu") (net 9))
 (segment (start 37.5625 20.8775) (end 37.5625 20.5725) (width 0.25) (layer "F.Cu") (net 9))
 (segment (start 37.5625 21.1975) (end 37.5625 20.5725) (width 0.25) (layer "F.Cu") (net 9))
 (segment (start 35.7375 22.7025) (end 37.5625 20.8775) (width 0.25) (layer "F.Cu") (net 9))
 (segment (start 32.8375 10.1825) (end 37.3325 10.1825) (width 0.25) (layer "B.Cu") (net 8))
 (segment (start 32.3025 26.8825) (end 31.1675 25.7475) (width 0.25) (layer "B.Cu") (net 8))
 (segment (start 31.1675 11.8525) (end 32.8375 10.1825) (width 0.25) (layer "B.Cu") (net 8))
 (segment (start 37.3325 10.1825) (end 40.1025 12.9525) (width 0.25) (layer "B.Cu") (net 8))
 (segment (start 31.1675 25.7475) (end 31.1675 11.8525) (width 0.25) (layer "B.Cu") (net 8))
 (segment (start 33.6075 25.6475) (end 33.6075 11.5725) (width 0.25) (layer "B.Cu") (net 7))
 (segment (start 36.7175 10.8825) (end 37.5625 11.7275) (width 0.25) (layer "B.Cu") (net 7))
 (segment (start 33.6075 11.5725) (end 34.2975 10.8825) (width 0.25) (layer "B.Cu") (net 7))
 (segment (start 37.5625 11.7275) (end 37.5625 12.9525) (width 0.25) (layer "B.Cu") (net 7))
 (segment (start 34.2975 10.8825) (end 36.7175 10.8825) (width 0.25) (layer "B.Cu") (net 7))
 (segment (start 34.8425 26.8825) (end 33.6075 25.6475) (width 0.25) (layer "B.Cu") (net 7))
 (segment (start 35.0225 12.9525) (end 36.1475 14.0775) (width 0.25) (layer "B.Cu") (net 6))
 (segment (start 36.1475 25.6475) (end 37.3825 26.8825) (width 0.25) (layer "B.Cu") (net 6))
 (segment (start 36.1475 14.0775) (end 36.1475 25.6475) (width 0.25) (layer "B.Cu") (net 6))
 (segment (start 32.4825 16.3275) (end 32.4825 12.9525) (width 0.25) (layer "F.Cu") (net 5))
 (segment (start 37.6675 18.5225) (end 34.6775 18.5225) (width 0.25) (layer "F.Cu") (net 5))
 (segment (start 39.9225 23.1775) (end 38.7339 21.9889) (width 0.25) (layer "F.Cu") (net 5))
 (segment (start 38.7339 21.9889) (end 38.7339 19.5961) (width 0.25) (layer "F.Cu") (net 5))
 (segment (start 38.7339 19.5961) (end 38.7375 19.5925) (width 0.25) (layer "F.Cu") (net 5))
 (segment (start 34.6775 18.5225) (end 32.4825 16.3275) (width 0.25) (layer "F.Cu") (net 5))
 (segment (start 39.9225 26.8825) (end 39.9225 23.1775) (width 0.25) (layer "F.Cu") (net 5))
 (segment (start 38.7375 19.5925) (end 37.6675 18.5225) (width 0.25) (layer "F.Cu") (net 5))
 (segment (start 32.4175 10.7525) (end 35.8525 10.7525) (width 0.25) (layer "F.Cu") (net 4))
 (segment (start 35.8525 10.7525) (end 39.9425 6.6625) (width 0.25) (layer "F.Cu") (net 4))
 (segment (start 31.2175 11.9525) (end 32.4175 10.7525) (width 0.25) (layer "F.Cu") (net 4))
 (segment (start 40.1025 15.4875) (end 40.1025 20.5725) (width 0.25) (layer "F.Cu") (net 4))
 (segment (start 27.4025 20.5725) (end 27.4025 17.8175) (width 0.25) (layer "F.Cu") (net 4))
 (segment (start 13.3275 7.5625) (end 15.9475 4.9425) (width 0.25) (layer "F.Cu") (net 4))
 (segment (start 22.3225 20.5725) (end 24.8625 20.5725) (width 0.25) (layer "F.Cu") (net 4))
 (segment (start 25.7075 4.9425) (end 26.5275 4.9425) (width 0.25) (layer "F.Cu") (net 4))
 (segment (start 15.9475 4.9425) (end 25.7075 4.9425) (width 0.25) (layer "F.Cu") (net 4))
 (segment (start 31.2175 14.0025) (end 31.2175 11.9525) (width 0.25) (layer "F.Cu") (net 4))
 (segment (start 39.9425 6.6625) (end 38.7375 7.8675) (width 0.25) (layer "F.Cu") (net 4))
 (segment (start 19.6025 23.2925) (end 22.3225 20.5725) (width 0.25) (layer "F.Cu") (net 4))
 (segment (start 39.9425 6.6625) (end 38.2225 4.9425) (width 0.25) (layer "F.Cu") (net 4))
 (segment (start 27.4025 20.5725) (end 24.8625 20.5725) (width 0.25) (layer "F.Cu") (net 4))
 (segment (start 38.2225 4.9425) (end 25.7075 4.9425) (width 0.25) (layer "F.Cu") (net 4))
 (segment (start 19.6025 26.8825) (end 19.6025 23.2925) (width 0.25) (layer "F.Cu") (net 4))
 (segment (start 38.7375 7.8675) (end 38.7375 14.1225) (width 0.25) (layer "F.Cu") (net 4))
 (segment (start 26.5275 4.9425) (end 28.2475 6.6625) (width 0.25) (layer "F.Cu") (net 4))
 (segment (start 9.9975 7.5625) (end 13.3275 7.5625) (width 0.25) (layer "F.Cu") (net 4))
 (segment (start 38.7375 14.1225) (end 40.1025 15.4875) (width 0.25) (layer "F.Cu") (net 4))
 (segment (start 27.4025 17.8175) (end 31.2175 14.0025) (width 0.25) (layer "F.Cu") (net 4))
 (segment (start 17.6175 23.4725) (end 19.9075 21.1825) (width 0.25) (layer "F.Cu") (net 1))
 (segment (start 27.4025 14.7975) (end 27.4025 12.9525) (width 0.25) (layer "F.Cu") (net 1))
 (segment (start 19.9075 18.8725) (end 21.9075 16.8725) (width 0.25) (layer "F.Cu") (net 1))
 (segment (start 19.9075 21.1825) (end 19.9075 18.8725) (width 0.25) (layer "F.Cu") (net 1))
 (segment (start 25.3275 16.8725) (end 27.4025 14.7975) (width 0.25) (layer "F.Cu") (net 1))
 (segment (start 21.9075 16.8725) (end 25.3275 16.8725) (width 0.25) (layer "F.Cu") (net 1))
 (segment (start 32.3225 6.6625) (end 27.4025 11.5825) (width 0.25) (layer "B.Cu") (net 1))
 (segment (start 25.7325 14.6225) (end 27.4025 12.9525) (width 0.25) (layer "B.Cu") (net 1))
 (segment (start 20.6275 6.6625) (end 23.6575 9.6925) (width 0.25) (layer "B.Cu") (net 1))
 (segment (start 27.4025 11.5825) (end 27.4025 12.9525) (width 0.25) (layer "B.Cu") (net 1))
 (segment (start 23.6575 14.0225) (end 24.2575 14.6225) (width 0.25) (layer "B.Cu") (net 1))
 (segment (start 24.2575 14.6225) (end 25.7325 14.6225) (width 0.25) (layer "B.Cu") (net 1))
 (segment (start 23.6575 9.6925) (end 23.6575 14.0225) (width 0.25) (layer "B.Cu") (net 1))
 (segment (start 17.6175 19.495) (end 20.7 16.4125) (width 0.25) (layer "F.Cu") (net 2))
 (segment (start 23.2275 16.4125) (end 24.8625 14.7775) (width 0.25) (layer "F.Cu") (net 2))
 (segment (start 24.8625 14.7775) (end 24.8625 12.9525) (width 0.25) (layer "F.Cu") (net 2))
 (segment (start 20.7 16.4125) (end 23.2275 16.4125) (width 0.25) (layer "F.Cu") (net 2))
 (segment (start 23.1675 6.6625) (end 24.3425 5.4875) (width 0.25) (layer "B.Cu") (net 2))
 (segment (start 24.8625 8.3575) (end 23.1675 6.6625) (width 0.25) (layer "B.Cu") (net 2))
 (segment (start 33.6875 5.4875) (end 34.8625 6.6625) (width 0.25) (layer "B.Cu") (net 2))
 (segment (start 24.3425 5.4875) (end 33.6875 5.4875) (width 0.25) (layer "B.Cu") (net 2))
 (segment (start 24.8625 12.9525) (end 24.8625 8.3575) (width 0.25) (layer "B.Cu") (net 2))
 (segment (start 9.9975 19.495) (end 9.9975 23.4725) (width 0.25) (layer "F.Cu") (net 3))
 (segment (start 15.5825 17.5525) (end 11.4375 17.5525) (width 0.25) (layer "F.Cu") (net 3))
 (segment (start 23.4475 11.8925) (end 23.4475 15.1025) (width 0.25) (layer "F.Cu") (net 3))
 (segment (start 24.4775 10.8625) (end 23.4475 11.8925) (width 0.25) (layer "F.Cu") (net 3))
 (segment (start 11.4375 17.5525) (end 9.9975 18.9925) (width 0.25) (layer "F.Cu") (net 3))
 (segment (start 37.4025 6.6625) (end 34.0525 10.0125) (width 0.25) (layer "F.Cu") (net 3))
 (segment (start 25.7075 9.6325) (end 24.4775 10.8625) (width 0.25) (layer "F.Cu") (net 3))
 (segment (start 17.6175 15.5175) (end 15.5825 17.5525) (width 0.25) (layer "F.Cu") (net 3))
 (segment (start 34.0525 10.0125) (end 25.3275 10.0125) (width 0.25) (layer "F.Cu") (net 3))
 (segment (start 23.0325 15.5175) (end 17.6175 15.5175) (width 0.25) (layer "F.Cu") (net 3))
 (segment (start 25.3275 10.0125) (end 24.4775 10.8625) (width 0.25) (layer "F.Cu") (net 3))
 (segment (start 25.7075 6.6625) (end 25.7075 9.6325) (width 0.25) (layer "F.Cu") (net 3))
 (segment (start 23.4475 15.1025) (end 23.0325 15.5175) (width 0.25) (layer "F.Cu") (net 3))
 (segment (start 9.9975 18.9925) (end 9.9975 19.495) (width 0.25) (layer "F.Cu") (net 3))
 (segment (start 11.825 9.7125) (end 15.4675 9.7125) (width 0.25) (layer "F.Cu") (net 14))
 (segment (start 15.4675 9.7125) (end 17.6175 7.5625) (width 0.25) (layer "F.Cu") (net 14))
 (segment (start 9.9975 11.54) (end 11.825 9.7125) (width 0.25) (layer "F.Cu") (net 14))
 (segment (start 22.3225 12.9525) (end 22.3225 12.2675) (width 0.25) (layer "F.Cu") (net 14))
 (segment (start 22.3225 12.2675) (end 17.6175 7.5625) (width 0.25) (layer "F.Cu") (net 14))
 (segment (start 15.605 13.5525) (end 17.6175 11.54) (width 0.25) (layer "F.Cu") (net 13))
 (segment (start 9.9975 15.5175) (end 11.9625 13.5525) (width 0.25) (layer "F.Cu") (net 13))
 (segment (start 11.9625 13.5525) (end 15.605 13.5525) (width 0.25) (layer "F.Cu") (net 13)))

